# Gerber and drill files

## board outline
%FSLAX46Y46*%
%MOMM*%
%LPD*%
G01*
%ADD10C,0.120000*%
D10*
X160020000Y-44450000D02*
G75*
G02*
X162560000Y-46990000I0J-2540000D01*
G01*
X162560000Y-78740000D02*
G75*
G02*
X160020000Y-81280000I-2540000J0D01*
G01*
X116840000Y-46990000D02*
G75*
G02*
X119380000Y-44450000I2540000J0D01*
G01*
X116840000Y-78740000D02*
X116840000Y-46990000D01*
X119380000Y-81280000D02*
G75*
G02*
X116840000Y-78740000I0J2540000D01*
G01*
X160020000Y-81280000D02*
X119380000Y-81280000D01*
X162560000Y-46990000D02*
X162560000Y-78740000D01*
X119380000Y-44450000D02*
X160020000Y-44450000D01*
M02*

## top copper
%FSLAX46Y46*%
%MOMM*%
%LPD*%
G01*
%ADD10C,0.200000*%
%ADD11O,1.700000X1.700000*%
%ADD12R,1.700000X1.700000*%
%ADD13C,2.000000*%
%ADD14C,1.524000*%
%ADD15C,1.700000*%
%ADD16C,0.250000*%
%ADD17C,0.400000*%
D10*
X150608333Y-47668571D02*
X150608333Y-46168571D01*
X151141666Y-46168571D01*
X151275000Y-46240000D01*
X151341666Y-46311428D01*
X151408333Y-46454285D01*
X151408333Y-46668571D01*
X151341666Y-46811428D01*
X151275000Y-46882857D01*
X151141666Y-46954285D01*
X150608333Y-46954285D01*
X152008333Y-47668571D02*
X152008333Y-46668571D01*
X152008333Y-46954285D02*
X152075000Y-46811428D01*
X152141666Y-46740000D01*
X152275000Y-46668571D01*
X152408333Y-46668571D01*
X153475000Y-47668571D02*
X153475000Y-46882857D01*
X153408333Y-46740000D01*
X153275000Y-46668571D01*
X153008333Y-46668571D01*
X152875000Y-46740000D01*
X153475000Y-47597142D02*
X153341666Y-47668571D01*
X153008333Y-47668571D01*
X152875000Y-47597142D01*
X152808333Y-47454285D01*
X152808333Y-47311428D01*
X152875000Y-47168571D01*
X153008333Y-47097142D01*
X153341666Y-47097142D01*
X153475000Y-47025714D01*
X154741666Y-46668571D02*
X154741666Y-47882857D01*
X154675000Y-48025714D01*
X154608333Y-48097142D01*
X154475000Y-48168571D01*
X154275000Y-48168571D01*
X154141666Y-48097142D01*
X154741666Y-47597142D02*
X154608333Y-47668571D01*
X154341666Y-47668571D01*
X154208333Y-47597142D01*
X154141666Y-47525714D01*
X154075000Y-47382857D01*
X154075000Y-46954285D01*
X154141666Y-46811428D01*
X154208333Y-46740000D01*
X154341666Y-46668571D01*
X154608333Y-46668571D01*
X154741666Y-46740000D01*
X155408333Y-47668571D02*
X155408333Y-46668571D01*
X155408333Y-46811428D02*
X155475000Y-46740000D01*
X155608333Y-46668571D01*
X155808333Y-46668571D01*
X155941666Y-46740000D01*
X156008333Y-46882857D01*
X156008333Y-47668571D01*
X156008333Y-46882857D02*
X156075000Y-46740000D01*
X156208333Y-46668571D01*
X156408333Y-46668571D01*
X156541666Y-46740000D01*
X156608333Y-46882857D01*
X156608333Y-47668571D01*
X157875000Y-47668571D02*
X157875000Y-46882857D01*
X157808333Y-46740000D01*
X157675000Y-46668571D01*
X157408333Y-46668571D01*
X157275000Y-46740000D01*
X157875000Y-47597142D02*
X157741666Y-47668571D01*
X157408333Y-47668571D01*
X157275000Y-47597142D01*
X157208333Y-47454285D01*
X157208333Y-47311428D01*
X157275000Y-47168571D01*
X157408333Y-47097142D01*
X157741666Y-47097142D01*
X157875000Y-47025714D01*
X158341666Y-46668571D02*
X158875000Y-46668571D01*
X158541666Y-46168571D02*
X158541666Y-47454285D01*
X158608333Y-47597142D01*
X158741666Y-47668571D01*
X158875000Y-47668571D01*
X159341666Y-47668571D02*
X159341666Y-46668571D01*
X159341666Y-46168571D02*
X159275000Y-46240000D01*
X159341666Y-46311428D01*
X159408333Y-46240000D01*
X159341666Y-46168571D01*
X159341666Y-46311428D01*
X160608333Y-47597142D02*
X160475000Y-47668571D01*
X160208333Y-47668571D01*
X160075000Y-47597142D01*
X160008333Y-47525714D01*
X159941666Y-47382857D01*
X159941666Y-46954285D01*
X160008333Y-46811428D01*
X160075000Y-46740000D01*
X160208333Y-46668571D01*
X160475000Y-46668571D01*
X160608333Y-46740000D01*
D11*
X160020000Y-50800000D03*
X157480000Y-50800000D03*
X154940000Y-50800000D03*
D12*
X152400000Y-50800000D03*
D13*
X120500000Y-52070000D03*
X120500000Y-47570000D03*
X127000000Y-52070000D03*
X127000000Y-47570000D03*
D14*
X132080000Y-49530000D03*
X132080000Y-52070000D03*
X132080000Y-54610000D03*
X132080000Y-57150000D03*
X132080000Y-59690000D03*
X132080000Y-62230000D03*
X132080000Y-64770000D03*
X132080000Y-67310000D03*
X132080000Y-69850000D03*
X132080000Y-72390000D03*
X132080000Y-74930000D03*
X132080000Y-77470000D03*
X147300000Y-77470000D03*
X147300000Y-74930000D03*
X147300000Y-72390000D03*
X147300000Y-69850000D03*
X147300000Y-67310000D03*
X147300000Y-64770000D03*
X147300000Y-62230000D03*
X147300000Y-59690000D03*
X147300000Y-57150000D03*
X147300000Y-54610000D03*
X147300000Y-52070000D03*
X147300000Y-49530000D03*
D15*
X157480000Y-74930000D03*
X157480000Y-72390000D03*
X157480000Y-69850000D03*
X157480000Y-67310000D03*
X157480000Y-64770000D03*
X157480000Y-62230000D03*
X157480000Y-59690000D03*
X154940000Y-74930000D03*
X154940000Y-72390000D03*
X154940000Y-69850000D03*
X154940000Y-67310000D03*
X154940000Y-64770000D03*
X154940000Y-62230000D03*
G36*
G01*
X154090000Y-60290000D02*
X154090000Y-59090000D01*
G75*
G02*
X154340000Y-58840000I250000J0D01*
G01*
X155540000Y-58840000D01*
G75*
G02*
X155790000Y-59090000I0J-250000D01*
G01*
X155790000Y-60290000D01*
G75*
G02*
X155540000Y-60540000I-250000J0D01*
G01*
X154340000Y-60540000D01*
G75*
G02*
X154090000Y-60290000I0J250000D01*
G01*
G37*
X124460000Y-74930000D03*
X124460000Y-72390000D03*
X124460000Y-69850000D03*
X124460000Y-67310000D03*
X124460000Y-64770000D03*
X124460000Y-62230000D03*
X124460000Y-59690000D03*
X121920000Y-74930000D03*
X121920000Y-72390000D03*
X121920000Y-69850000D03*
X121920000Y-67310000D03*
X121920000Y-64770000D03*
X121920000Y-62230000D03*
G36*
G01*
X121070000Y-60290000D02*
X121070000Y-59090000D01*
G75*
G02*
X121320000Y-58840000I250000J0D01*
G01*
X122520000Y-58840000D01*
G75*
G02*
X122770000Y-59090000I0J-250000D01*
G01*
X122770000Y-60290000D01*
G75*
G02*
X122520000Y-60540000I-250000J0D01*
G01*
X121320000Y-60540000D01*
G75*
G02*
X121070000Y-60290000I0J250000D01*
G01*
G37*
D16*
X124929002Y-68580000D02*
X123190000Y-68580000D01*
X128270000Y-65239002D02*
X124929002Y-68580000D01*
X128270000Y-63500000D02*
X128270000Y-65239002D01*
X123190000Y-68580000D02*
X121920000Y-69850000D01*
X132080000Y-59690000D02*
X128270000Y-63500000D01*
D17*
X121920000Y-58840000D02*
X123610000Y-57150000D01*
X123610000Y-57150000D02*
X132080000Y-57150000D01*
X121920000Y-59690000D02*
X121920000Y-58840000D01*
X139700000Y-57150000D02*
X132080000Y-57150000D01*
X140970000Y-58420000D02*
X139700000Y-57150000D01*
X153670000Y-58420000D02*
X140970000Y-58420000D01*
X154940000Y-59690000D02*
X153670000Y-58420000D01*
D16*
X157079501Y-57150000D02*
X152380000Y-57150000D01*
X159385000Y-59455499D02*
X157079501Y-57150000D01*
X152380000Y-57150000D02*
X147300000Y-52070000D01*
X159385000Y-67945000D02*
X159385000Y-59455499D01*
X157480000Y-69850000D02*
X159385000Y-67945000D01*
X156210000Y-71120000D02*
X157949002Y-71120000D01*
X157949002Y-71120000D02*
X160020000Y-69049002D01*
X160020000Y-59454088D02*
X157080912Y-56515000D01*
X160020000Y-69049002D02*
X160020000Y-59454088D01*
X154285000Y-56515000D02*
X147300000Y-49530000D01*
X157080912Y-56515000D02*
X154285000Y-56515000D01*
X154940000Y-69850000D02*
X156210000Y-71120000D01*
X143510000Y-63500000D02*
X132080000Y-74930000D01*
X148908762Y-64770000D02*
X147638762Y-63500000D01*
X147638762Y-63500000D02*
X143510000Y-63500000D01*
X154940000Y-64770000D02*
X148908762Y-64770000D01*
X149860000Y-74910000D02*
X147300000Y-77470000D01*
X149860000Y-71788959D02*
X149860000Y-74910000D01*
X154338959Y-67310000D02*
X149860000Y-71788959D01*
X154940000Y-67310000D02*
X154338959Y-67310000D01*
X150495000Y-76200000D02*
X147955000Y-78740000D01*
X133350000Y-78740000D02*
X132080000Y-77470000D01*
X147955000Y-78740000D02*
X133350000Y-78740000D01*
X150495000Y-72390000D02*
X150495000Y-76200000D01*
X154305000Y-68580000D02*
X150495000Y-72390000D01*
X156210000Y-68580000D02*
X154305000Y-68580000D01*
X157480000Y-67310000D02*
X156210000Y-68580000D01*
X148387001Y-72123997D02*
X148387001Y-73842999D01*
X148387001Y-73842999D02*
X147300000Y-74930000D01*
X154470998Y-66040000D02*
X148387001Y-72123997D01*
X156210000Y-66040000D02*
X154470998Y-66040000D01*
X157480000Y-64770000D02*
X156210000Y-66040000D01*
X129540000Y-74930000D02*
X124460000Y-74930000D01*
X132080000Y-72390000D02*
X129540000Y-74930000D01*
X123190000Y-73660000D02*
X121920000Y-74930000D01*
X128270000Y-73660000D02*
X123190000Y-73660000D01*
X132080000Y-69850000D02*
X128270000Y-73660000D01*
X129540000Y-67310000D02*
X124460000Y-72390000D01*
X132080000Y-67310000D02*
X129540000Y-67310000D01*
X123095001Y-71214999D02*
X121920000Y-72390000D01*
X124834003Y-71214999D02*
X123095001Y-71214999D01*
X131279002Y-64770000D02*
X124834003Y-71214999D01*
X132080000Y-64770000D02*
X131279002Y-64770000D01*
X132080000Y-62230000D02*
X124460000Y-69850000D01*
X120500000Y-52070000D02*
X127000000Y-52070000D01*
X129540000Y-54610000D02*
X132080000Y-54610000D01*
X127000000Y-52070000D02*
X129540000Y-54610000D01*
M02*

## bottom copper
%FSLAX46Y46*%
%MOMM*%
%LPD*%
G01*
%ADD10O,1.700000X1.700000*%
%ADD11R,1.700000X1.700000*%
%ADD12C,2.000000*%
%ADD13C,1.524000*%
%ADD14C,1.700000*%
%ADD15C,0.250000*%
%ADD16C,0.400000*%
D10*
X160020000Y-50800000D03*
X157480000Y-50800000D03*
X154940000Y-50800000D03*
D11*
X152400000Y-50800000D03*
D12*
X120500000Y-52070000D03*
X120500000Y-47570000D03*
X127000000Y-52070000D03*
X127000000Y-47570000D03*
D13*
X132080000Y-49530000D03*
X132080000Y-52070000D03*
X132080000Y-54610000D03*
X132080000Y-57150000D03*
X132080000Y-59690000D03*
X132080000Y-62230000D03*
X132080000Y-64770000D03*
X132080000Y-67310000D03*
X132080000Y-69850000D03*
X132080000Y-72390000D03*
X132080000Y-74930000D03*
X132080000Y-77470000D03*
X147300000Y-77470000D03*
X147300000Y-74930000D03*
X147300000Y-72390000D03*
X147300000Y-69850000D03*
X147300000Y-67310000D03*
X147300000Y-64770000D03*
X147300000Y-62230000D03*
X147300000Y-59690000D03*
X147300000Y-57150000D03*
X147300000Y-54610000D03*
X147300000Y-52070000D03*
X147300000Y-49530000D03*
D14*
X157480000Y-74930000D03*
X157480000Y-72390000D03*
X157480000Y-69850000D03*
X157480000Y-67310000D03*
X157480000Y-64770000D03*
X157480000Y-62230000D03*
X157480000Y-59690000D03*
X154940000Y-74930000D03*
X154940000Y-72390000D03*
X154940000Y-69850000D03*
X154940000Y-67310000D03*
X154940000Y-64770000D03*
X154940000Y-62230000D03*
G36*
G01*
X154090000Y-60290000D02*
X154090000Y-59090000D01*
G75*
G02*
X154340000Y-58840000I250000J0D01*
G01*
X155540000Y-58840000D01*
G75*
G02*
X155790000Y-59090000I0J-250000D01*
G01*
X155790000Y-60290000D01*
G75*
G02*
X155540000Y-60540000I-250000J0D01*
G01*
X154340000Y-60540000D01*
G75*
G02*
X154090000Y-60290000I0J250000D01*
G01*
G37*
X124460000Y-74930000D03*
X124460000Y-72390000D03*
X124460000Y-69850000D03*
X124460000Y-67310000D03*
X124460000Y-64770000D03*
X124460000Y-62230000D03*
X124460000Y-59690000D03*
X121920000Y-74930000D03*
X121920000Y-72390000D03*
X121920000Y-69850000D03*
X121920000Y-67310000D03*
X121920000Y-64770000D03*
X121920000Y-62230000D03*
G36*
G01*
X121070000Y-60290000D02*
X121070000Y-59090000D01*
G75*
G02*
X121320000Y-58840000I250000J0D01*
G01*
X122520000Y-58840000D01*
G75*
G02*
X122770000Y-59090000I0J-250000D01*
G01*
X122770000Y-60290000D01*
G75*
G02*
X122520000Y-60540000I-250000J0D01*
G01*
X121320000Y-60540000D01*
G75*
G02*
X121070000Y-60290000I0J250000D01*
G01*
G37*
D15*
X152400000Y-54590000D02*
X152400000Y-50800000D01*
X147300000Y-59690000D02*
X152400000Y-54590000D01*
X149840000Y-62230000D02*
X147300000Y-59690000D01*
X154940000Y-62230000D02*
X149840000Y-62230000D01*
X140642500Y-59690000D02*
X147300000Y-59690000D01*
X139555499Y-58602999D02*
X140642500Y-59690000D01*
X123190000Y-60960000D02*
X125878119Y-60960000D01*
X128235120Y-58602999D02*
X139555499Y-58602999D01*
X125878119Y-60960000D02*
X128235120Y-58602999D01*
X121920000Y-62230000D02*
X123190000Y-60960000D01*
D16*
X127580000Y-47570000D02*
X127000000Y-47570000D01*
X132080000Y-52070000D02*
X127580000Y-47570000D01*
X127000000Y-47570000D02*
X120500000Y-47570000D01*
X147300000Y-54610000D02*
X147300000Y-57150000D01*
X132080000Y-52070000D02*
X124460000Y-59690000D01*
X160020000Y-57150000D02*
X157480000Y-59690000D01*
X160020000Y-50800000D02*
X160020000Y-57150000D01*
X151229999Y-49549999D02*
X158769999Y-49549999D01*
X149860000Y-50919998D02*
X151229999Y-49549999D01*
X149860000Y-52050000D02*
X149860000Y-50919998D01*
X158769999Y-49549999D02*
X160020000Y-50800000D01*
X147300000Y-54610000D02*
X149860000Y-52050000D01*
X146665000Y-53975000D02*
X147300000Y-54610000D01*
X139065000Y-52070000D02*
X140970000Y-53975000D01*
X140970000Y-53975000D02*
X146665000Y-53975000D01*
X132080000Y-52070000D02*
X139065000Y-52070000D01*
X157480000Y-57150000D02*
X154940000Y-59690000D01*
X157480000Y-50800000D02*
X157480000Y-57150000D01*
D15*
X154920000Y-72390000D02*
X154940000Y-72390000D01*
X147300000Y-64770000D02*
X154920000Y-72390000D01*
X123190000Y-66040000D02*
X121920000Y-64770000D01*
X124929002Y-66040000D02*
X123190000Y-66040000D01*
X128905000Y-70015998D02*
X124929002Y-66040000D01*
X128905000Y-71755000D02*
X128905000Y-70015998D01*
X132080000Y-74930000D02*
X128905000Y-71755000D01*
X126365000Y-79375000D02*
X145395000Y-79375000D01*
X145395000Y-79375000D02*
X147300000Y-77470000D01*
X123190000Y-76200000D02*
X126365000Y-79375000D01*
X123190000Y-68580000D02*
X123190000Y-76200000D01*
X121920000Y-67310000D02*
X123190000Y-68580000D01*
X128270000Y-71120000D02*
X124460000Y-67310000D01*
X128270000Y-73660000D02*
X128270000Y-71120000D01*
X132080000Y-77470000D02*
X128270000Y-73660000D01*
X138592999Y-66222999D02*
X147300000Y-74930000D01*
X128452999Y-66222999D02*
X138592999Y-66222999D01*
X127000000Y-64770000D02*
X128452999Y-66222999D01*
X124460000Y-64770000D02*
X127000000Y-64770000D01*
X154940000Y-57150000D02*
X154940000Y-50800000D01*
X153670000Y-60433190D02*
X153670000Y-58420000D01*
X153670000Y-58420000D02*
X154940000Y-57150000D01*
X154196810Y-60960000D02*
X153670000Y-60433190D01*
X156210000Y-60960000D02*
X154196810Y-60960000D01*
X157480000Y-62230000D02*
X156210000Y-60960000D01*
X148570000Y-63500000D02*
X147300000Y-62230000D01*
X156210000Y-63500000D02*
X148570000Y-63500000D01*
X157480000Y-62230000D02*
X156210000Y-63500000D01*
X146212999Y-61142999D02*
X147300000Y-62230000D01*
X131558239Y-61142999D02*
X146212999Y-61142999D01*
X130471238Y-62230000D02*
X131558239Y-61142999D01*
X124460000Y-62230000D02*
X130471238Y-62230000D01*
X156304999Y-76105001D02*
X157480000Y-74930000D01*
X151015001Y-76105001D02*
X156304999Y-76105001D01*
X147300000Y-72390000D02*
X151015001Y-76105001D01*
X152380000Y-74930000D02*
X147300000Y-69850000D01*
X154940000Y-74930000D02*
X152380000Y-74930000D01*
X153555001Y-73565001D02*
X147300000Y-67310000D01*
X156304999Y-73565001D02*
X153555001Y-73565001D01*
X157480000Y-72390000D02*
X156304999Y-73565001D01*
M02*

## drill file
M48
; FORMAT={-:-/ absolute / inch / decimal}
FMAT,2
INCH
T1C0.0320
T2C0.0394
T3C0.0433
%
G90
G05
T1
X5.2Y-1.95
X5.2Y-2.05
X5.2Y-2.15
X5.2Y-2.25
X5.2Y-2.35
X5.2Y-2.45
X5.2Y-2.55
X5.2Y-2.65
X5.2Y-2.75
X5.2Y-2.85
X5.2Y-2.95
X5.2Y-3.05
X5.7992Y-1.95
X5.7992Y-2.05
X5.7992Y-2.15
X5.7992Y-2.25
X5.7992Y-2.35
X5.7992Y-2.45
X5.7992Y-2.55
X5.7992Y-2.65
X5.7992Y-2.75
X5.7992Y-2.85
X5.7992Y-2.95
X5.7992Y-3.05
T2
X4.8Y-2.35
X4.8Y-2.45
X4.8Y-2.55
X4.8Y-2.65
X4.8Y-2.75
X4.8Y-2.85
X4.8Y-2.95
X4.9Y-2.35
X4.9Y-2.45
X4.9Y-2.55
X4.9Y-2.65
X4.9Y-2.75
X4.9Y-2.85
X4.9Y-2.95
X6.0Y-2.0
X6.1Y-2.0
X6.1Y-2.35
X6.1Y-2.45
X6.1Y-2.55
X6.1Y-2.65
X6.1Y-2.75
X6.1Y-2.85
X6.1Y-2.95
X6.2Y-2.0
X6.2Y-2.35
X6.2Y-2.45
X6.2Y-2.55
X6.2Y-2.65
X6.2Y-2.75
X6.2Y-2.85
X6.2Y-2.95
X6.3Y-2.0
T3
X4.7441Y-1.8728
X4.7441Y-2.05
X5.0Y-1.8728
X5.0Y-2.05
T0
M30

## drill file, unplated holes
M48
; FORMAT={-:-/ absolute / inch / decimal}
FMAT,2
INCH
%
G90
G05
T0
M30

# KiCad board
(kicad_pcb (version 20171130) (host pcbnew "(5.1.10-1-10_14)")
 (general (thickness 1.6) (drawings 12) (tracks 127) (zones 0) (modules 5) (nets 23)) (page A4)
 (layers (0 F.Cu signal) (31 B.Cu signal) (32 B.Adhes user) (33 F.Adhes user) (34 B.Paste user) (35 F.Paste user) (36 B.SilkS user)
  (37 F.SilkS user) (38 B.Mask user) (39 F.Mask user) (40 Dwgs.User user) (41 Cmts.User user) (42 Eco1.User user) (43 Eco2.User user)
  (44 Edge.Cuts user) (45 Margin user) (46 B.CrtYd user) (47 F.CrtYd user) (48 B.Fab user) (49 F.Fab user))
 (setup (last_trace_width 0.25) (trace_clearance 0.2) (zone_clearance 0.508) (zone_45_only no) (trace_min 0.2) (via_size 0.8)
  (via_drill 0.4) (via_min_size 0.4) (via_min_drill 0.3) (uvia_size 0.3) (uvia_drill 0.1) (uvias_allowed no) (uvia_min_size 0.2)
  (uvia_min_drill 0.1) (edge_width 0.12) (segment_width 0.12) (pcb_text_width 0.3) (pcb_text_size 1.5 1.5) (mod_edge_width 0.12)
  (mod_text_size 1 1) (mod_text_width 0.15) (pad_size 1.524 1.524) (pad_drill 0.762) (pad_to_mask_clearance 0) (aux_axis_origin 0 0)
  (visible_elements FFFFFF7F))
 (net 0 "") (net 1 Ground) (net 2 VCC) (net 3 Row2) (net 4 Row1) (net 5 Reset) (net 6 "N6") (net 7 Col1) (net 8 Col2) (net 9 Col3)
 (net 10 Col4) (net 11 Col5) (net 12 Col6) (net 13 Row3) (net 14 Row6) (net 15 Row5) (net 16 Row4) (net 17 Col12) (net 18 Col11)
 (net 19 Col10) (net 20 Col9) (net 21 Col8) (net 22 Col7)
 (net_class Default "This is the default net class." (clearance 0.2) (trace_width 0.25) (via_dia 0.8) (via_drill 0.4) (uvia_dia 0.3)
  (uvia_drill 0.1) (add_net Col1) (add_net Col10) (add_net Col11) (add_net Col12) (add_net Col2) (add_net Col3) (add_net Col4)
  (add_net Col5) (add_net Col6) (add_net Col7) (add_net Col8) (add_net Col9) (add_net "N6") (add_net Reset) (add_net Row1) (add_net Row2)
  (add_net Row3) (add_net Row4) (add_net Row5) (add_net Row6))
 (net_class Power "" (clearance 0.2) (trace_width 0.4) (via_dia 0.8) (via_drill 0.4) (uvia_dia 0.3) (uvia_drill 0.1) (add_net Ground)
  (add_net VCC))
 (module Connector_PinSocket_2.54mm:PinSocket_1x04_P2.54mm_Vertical (layer F.Cu) (at 152.4 50.8 90)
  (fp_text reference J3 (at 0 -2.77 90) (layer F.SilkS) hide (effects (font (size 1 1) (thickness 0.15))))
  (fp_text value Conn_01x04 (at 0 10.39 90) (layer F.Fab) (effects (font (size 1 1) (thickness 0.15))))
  (pad 4 thru_hole oval (at 0 7.62 90) (size 1.7 1.7) (drill 1) (layers *.Cu *.Mask) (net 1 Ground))
  (pad 3 thru_hole oval (at 0 5.08 90) (size 1.7 1.7) (drill 1) (layers *.Cu *.Mask) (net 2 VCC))
  (pad 2 thru_hole oval (at 0 2.54 90) (size 1.7 1.7) (drill 1) (layers *.Cu *.Mask) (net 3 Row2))
  (pad 1 thru_hole rect (at 0 0 90) (size 1.7 1.7) (drill 1) (layers *.Cu *.Mask) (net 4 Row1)))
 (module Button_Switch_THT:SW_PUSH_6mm (layer F.Cu) (at 127 52.07 180)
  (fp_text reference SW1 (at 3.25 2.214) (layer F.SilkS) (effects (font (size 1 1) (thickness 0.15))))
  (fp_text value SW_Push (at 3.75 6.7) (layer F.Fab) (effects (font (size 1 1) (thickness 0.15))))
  (pad 1 thru_hole circle (at 6.5 0 270) (size 2 2) (drill 1.1) (layers *.Cu *.Mask) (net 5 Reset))
  (pad 2 thru_hole circle (at 6.5 4.5 270) (size 2 2) (drill 1.1) (layers *.Cu *.Mask) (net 1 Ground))
  (pad 1 thru_hole circle (at 0 0 270) (size 2 2) (drill 1.1) (layers *.Cu *.Mask) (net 5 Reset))
  (pad 2 thru_hole circle (at 0 4.5 270) (size 2 2) (drill 1.1) (layers *.Cu *.Mask) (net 1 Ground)))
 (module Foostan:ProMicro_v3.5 (layer F.Cu) (at 139.6886 64.008)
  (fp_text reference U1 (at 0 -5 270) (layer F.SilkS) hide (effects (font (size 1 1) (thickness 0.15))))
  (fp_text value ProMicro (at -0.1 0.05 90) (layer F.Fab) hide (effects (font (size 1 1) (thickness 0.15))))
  (pad 24 thru_hole circle (at -7.6086 -14.478) (size 1.524 1.524) (drill 0.8128) (layers *.Cu F.SilkS B.Mask) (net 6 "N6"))
  (pad 23 thru_hole circle (at -7.6086 -11.938) (size 1.524 1.524) (drill 0.8128) (layers *.Cu F.SilkS B.Mask) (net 1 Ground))
  (pad 22 thru_hole circle (at -7.6086 -9.398) (size 1.524 1.524) (drill 0.8128) (layers *.Cu F.SilkS B.Mask) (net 5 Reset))
  (pad 21 thru_hole circle (at -7.6086 -6.858) (size 1.524 1.524) (drill 0.8128) (layers *.Cu F.SilkS B.Mask) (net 2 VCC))
  (pad 20 thru_hole circle (at -7.6086 -4.318) (size 1.524 1.524) (drill 0.8128) (layers *.Cu F.SilkS B.Mask) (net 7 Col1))
  (pad 19 thru_hole circle (at -7.6086 -1.778) (size 1.524 1.524) (drill 0.8128) (layers *.Cu F.SilkS B.Mask) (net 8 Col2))
  (pad 18 thru_hole circle (at -7.6086 0.762) (size 1.524 1.524) (drill 0.8128) (layers *.Cu F.SilkS B.Mask) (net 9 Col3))
  (pad 17 thru_hole circle (at -7.6086 3.302) (size 1.524 1.524) (drill 0.8128) (layers *.Cu F.SilkS B.Mask) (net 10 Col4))
  (pad 16 thru_hole circle (at -7.6086 5.842) (size 1.524 1.524) (drill 0.8128) (layers *.Cu F.SilkS B.Mask) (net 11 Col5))
  (pad 15 thru_hole circle (at -7.6086 8.382) (size 1.524 1.524) (drill 0.8128) (layers *.Cu F.SilkS B.Mask) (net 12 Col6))
  (pad 14 thru_hole circle (at -7.6086 10.922) (size 1.524 1.524) (drill 0.8128) (layers *.Cu F.SilkS B.Mask) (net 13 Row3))
  (pad 13 thru_hole circle (at -7.6086 13.462) (size 1.524 1.524) (drill 0.8128) (layers *.Cu F.SilkS B.Mask) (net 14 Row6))
  (pad 12 thru_hole circle (at 7.6114 13.462) (size 1.524 1.524) (drill 0.8128) (layers *.Cu F.SilkS B.Mask) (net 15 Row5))
  (pad 11 thru_hole circle (at 7.6114 10.922) (size 1.524 1.524) (drill 0.8128) (layers *.Cu F.SilkS B.Mask) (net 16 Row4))
  (pad 10 thru_hole circle (at 7.6114 8.382) (size 1.524 1.524) (drill 0.8128) (layers *.Cu F.SilkS B.Mask) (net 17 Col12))
  (pad 9 thru_hole circle (at 7.6114 5.842) (size 1.524 1.524) (drill 0.8128) (layers *.Cu F.SilkS B.Mask) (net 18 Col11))
  (pad 8 thru_hole circle (at 7.6114 3.302) (size 1.524 1.524) (drill 0.8128) (layers *.Cu F.SilkS B.Mask) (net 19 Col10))
  (pad 7 thru_hole circle (at 7.6114 0.762) (size 1.524 1.524) (drill 0.8128) (layers *.Cu F.SilkS B.Mask) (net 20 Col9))
  (pad 6 thru_hole circle (at 7.6114 -1.778) (size 1.524 1.524) (drill 0.8128) (layers *.Cu F.SilkS B.Mask) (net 3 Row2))
  (pad 5 thru_hole circle (at 7.6114 -4.318) (size 1.524 1.524) (drill 0.8128) (layers *.Cu F.SilkS B.Mask) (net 4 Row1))
  (pad 4 thru_hole circle (at 7.6114 -6.858) (size 1.524 1.524) (drill 0.8128) (layers *.Cu F.SilkS B.Mask) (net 1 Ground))
  (pad 3 thru_hole circle (at 7.6114 -9.398) (size 1.524 1.524) (drill 0.8128) (layers *.Cu F.SilkS B.Mask) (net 1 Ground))
  (pad 2 thru_hole circle (at 7.6114 -11.938) (size 1.524 1.524) (drill 0.8128) (layers *.Cu F.SilkS B.Mask) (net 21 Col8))
  (pad 1 thru_hole circle (at 7.6114 -14.478) (size 1.524 1.524) (drill 0.8128) (layers *.Cu F.SilkS B.Mask) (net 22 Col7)))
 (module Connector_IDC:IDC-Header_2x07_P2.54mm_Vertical (layer F.Cu) (at 154.94 59.69)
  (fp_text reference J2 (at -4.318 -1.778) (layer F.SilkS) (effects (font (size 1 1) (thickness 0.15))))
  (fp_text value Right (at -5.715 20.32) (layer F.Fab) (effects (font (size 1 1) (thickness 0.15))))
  (pad 14 thru_hole circle (at 2.54 15.24) (size 1.7 1.7) (drill 1) (layers *.Cu *.Mask) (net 17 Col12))
  (pad 12 thru_hole circle (at 2.54 12.7) (size 1.7 1.7) (drill 1) (layers *.Cu *.Mask) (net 19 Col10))
  (pad 10 thru_hole circle (at 2.54 10.16) (size 1.7 1.7) (drill 1) (layers *.Cu *.Mask) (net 21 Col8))
  (pad 8 thru_hole circle (at 2.54 7.62) (size 1.7 1.7) (drill 1) (layers *.Cu *.Mask) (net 14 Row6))
  (pad 6 thru_hole circle (at 2.54 5.08) (size 1.7 1.7) (drill 1) (layers *.Cu *.Mask) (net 16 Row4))
  (pad 4 thru_hole circle (at 2.54 2.54) (size 1.7 1.7) (drill 1) (layers *.Cu *.Mask) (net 3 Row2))
  (pad 2 thru_hole circle (at 2.54 0) (size 1.7 1.7) (drill 1) (layers *.Cu *.Mask) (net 1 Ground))
  (pad 13 thru_hole circle (at 0 15.24) (size 1.7 1.7) (drill 1) (layers *.Cu *.Mask) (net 18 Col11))
  (pad 11 thru_hole circle (at 0 12.7) (size 1.7 1.7) (drill 1) (layers *.Cu *.Mask) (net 20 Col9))
  (pad 9 thru_hole circle (at 0 10.16) (size 1.7 1.7) (drill 1) (layers *.Cu *.Mask) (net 22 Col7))
  (pad 7 thru_hole circle (at 0 7.62) (size 1.7 1.7) (drill 1) (layers *.Cu *.Mask) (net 15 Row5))
  (pad 5 thru_hole circle (at 0 5.08) (size 1.7 1.7) (drill 1) (layers *.Cu *.Mask) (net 13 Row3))
  (pad 3 thru_hole circle (at 0 2.54) (size 1.7 1.7) (drill 1) (layers *.Cu *.Mask) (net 4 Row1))
  (pad 1 thru_hole roundrect (at 0 0) (size 1.7 1.7) (drill 1) (layers *.Cu *.Mask) (roundrect_rratio 0.1470588235294118) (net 2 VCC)))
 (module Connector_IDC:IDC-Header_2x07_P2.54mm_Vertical (layer F.Cu) (at 121.92 59.69)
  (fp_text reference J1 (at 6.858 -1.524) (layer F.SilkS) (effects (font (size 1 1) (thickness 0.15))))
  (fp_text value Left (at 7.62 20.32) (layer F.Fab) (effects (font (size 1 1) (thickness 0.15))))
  (pad 14 thru_hole circle (at 2.54 15.24) (size 1.7 1.7) (drill 1) (layers *.Cu *.Mask) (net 12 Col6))
  (pad 12 thru_hole circle (at 2.54 12.7) (size 1.7 1.7) (drill 1) (layers *.Cu *.Mask) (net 10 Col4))
  (pad 10 thru_hole circle (at 2.54 10.16) (size 1.7 1.7) (drill 1) (layers *.Cu *.Mask) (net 8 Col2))
  (pad 8 thru_hole circle (at 2.54 7.62) (size 1.7 1.7) (drill 1) (layers *.Cu *.Mask) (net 14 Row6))
  (pad 6 thru_hole circle (at 2.54 5.08) (size 1.7 1.7) (drill 1) (layers *.Cu *.Mask) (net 16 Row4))
  (pad 4 thru_hole circle (at 2.54 2.54) (size 1.7 1.7) (drill 1) (layers *.Cu *.Mask) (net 3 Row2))
  (pad 2 thru_hole circle (at 2.54 0) (size 1.7 1.7) (drill 1) (layers *.Cu *.Mask) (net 1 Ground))
  (pad 13 thru_hole circle (at 0 15.24) (size 1.7 1.7) (drill 1) (layers *.Cu *.Mask) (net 11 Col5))
  (pad 11 thru_hole circle (at 0 12.7) (size 1.7 1.7) (drill 1) (layers *.Cu *.Mask) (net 9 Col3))
  (pad 9 thru_hole circle (at 0 10.16) (size 1.7 1.7) (drill 1) (layers *.Cu *.Mask) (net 7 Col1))
  (pad 7 thru_hole circle (at 0 7.62) (size 1.7 1.7) (drill 1) (layers *.Cu *.Mask) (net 15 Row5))
  (pad 5 thru_hole circle (at 0 5.08) (size 1.7 1.7) (drill 1) (layers *.Cu *.Mask) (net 13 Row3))
  (pad 3 thru_hole circle (at 0 2.54) (size 1.7 1.7) (drill 1) (layers *.Cu *.Mask) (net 4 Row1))
  (pad 1 thru_hole roundrect (at 0 0) (size 1.7 1.7) (drill 1) (layers *.Cu *.Mask) (roundrect_rratio 0.1470588235294118) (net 2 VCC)))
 (gr_arc (start 160.02 46.99) (end 162.56 46.99) (angle -90) (layer Edge.Cuts) (width 0.12))
 (gr_arc (start 160.02 78.74) (end 160.02 81.28) (angle -90) (layer Edge.Cuts) (width 0.12))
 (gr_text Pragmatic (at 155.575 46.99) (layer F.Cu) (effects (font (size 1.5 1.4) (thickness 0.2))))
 (gr_arc (start 119.38 46.99) (end 119.38 44.45) (angle -90) (layer Edge.Cuts) (width 0.12))
 (gr_line (start 116.84 78.74) (end 116.84 46.99) (layer Edge.Cuts) (width 0.12))
 (gr_arc (start 119.38 78.74) (end 116.84 78.74) (angle -90) (layer Edge.Cuts) (width 0.12))
 (gr_line (start 160.02 81.28) (end 119.38 81.28) (layer Edge.Cuts) (width 0.12))
 (gr_line (start 162.56 46.99) (end 162.56 78.74) (layer Edge.Cuts) (width 0.12))
 (gr_line (start 119.38 44.45) (end 160.02 44.45) (layer Edge.Cuts) (width 0.12))
 (segment (start 152.4 54.59) (end 152.4 50.8) (width 0.25) (layer B.Cu) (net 4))
 (segment (start 147.3 59.69) (end 152.4 54.59) (width 0.25) (layer B.Cu) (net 4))
 (segment (start 149.84 62.23) (end 147.3 59.69) (width 0.25) (layer B.Cu) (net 4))
 (segment (start 154.94 62.23) (end 149.84 62.23) (width 0.25) (layer B.Cu) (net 4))
 (segment (start 140.6425 59.69) (end 147.3 59.69) (width 0.25) (layer B.Cu) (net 4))
 (segment (start 139.555499 58.602999) (end 140.6425 59.69) (width 0.25) (layer B.Cu) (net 4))
 (segment (start 123.19 60.96) (end 125.878119 60.96) (width 0.25) (layer B.Cu) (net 4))
 (segment (start 128.23512 58.602999) (end 139.555499 58.602999) (width 0.25) (layer B.Cu) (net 4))
 (segment (start 125.878119 60.96) (end 128.23512 58.602999) (width 0.25) (layer B.Cu) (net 4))
 (segment (start 121.92 62.23) (end 123.19 60.96) (width 0.25) (layer B.Cu) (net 4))
 (segment (start 124.929002 68.58) (end 123.19 68.58) (width 0.25) (layer F.Cu) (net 7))
 (segment (start 128.27 65.239002) (end 124.929002 68.58) (width 0.25) (layer F.Cu) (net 7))
 (segment (start 128.27 63.5) (end 128.27 65.239002) (width 0.25) (layer F.Cu) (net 7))
 (segment (start 123.19 68.58) (end 121.92 69.85) (width 0.25) (layer F.Cu) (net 7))
 (segment (start 132.08 59.69) (end 128.27 63.5) (width 0.25) (layer F.Cu) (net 7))
 (segment (start 127.58 47.57) (end 127 47.57) (width 0.4) (layer B.Cu) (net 1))
 (segment (start 132.08 52.07) (end 127.58 47.57) (width 0.4) (layer B.Cu) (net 1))
 (segment (start 127 47.57) (end 120.5 47.57) (width 0.4) (layer B.Cu) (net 1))
 (segment (start 147.3 54.61) (end 147.3 57.15) (width 0.4) (layer B.Cu) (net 1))
 (segment (start 132.08 52.07) (end 124.46 59.69) (width 0.4) (layer B.Cu) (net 1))
 (segment (start 160.02 57.15) (end 157.48 59.69) (width 0.4) (layer B.Cu) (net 1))
 (segment (start 160.02 50.8) (end 160.02 57.15) (width 0.4) (layer B.Cu) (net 1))
 (segment (start 151.229999 49.549999) (end 158.769999 49.549999) (width 0.4) (layer B.Cu) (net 1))
 (segment (start 149.86 50.919998) (end 151.229999 49.549999) (width 0.4) (layer B.Cu) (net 1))
 (segment (start 149.86 52.05) (end 149.86 50.919998) (width 0.4) (layer B.Cu) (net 1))
 (segment (start 158.769999 49.549999) (end 160.02 50.8) (width 0.4) (layer B.Cu) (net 1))
 (segment (start 147.3 54.61) (end 149.86 52.05) (width 0.4) (layer B.Cu) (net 1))
 (segment (start 146.665 53.975) (end 147.3 54.61) (width 0.4) (layer B.Cu) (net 1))
 (segment (start 139.065 52.07) (end 140.97 53.975) (width 0.4) (layer B.Cu) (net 1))
 (segment (start 140.97 53.975) (end 146.665 53.975) (width 0.4) (layer B.Cu) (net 1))
 (segment (start 132.08 52.07) (end 139.065 52.07) (width 0.4) (layer B.Cu) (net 1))
 (segment (start 157.48 57.15) (end 154.94 59.69) (width 0.4) (layer B.Cu) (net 2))
 (segment (start 157.48 50.8) (end 157.48 57.15) (width 0.4) (layer B.Cu) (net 2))
 (segment (start 121.92 58.84) (end 123.61 57.15) (width 0.4) (layer F.Cu) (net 2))
 (segment (start 123.61 57.15) (end 132.08 57.15) (width 0.4) (layer F.Cu) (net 2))
 (segment (start 121.92 59.69) (end 121.92 58.84) (width 0.4) (layer F.Cu) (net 2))
 (segment (start 139.7 57.15) (end 132.08 57.15) (width 0.4) (layer F.Cu) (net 2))
 (segment (start 140.97 58.42) (end 139.7 57.15) (width 0.4) (layer F.Cu) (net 2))
 (segment (start 153.67 58.42) (end 140.97 58.42) (width 0.4) (layer F.Cu) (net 2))
 (segment (start 154.94 59.69) (end 153.67 58.42) (width 0.4) (layer F.Cu) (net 2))
 (segment (start 154.92 72.39) (end 154.94 72.39) (width 0.25) (layer B.Cu) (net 20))
 (segment (start 147.3 64.77) (end 154.92 72.39) (width 0.25) (layer B.Cu) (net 20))
 (segment (start 157.079501 57.15) (end 152.38 57.15) (width 0.25) (layer F.Cu) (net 21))
 (segment (start 159.385 59.455499) (end 157.079501 57.15) (width 0.25) (layer F.Cu) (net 21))
 (segment (start 152.38 57.15) (end 147.3 52.07) (width 0.25) (layer F.Cu) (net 21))
 (segment (start 159.385 67.945) (end 159.385 59.455499) (width 0.25) (layer F.Cu) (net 21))
 (segment (start 157.48 69.85) (end 159.385 67.945) (width 0.25) (layer F.Cu) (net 21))
 (segment (start 156.21 71.12) (end 157.949002 71.12) (width 0.25) (layer F.Cu) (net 22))
 (segment (start 157.949002 71.12) (end 160.02 69.049002) (width 0.25) (layer F.Cu) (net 22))
 (segment (start 160.02 59.454088) (end 157.080912 56.515) (width 0.25) (layer F.Cu) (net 22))
 (segment (start 160.02 69.049002) (end 160.02 59.454088) (width 0.25) (layer F.Cu) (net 22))
 (segment (start 154.285 56.515) (end 147.3 49.53) (width 0.25) (layer F.Cu) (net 22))
 (segment (start 157.080912 56.515) (end 154.285 56.515) (width 0.25) (layer F.Cu) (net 22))
 (segment (start 154.94 69.85) (end 156.21 71.12) (width 0.25) (layer F.Cu) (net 22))
 (segment (start 143.51 63.5) (end 132.08 74.93) (width 0.25) (layer F.Cu) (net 13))
 (segment (start 148.908762 64.77) (end 147.638762 63.5) (width 0.25) (layer F.Cu) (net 13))
 (segment (start 147.638762 63.5) (end 143.51 63.5) (width 0.25) (layer F.Cu) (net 13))
 (segment (start 154.94 64.77) (end 148.908762 64.77) (width 0.25) (layer F.Cu) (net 13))
 (segment (start 123.19 66.04) (end 121.92 64.77) (width 0.25) (layer B.Cu) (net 13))
 (segment (start 124.929002 66.04) (end 123.19 66.04) (width 0.25) (layer B.Cu) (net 13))
 (segment (start 128.905 70.015998) (end 124.929002 66.04) (width 0.25) (layer B.Cu) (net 13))
 (segment (start 128.905 71.755) (end 128.905 70.015998) (width 0.25) (layer B.Cu) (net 13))
 (segment (start 132.08 74.93) (end 128.905 71.755) (width 0.25) (layer B.Cu) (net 13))
 (segment (start 149.86 74.91) (end 147.3 77.47) (width 0.25) (layer F.Cu) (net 15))
 (segment (start 149.86 71.788959) (end 149.86 74.91) (width 0.25) (layer F.Cu) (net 15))
 (segment (start 154.338959 67.31) (end 149.86 71.788959) (width 0.25) (layer F.Cu) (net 15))
 (segment (start 154.94 67.31) (end 154.338959 67.31) (width 0.25) (layer F.Cu) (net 15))
 (segment (start 126.365 79.375) (end 145.395 79.375) (width 0.25) (layer B.Cu) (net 15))
 (segment (start 145.395 79.375) (end 147.3 77.47) (width 0.25) (layer B.Cu) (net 15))
 (segment (start 123.19 76.2) (end 126.365 79.375) (width 0.25) (layer B.Cu) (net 15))
 (segment (start 123.19 68.58) (end 123.19 76.2) (width 0.25) (layer B.Cu) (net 15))
 (segment (start 121.92 67.31) (end 123.19 68.58) (width 0.25) (layer B.Cu) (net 15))
 (segment (start 150.495 76.2) (end 147.955 78.74) (width 0.25) (layer F.Cu) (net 14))
 (segment (start 133.35 78.74) (end 132.08 77.47) (width 0.25) (layer F.Cu) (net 14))
 (segment (start 147.955 78.74) (end 133.35 78.74) (width 0.25) (layer F.Cu) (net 14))
 (segment (start 150.495 72.39) (end 150.495 76.2) (width 0.25) (layer F.Cu) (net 14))
 (segment (start 154.305 68.58) (end 150.495 72.39) (width 0.25) (layer F.Cu) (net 14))
 (segment (start 156.21 68.58) (end 154.305 68.58) (width 0.25) (layer F.Cu) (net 14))
 (segment (start 157.48 67.31) (end 156.21 68.58) (width 0.25) (layer F.Cu) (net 14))
 (segment (start 128.27 71.12) (end 124.46 67.31) (width 0.25) (layer B.Cu) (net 14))
 (segment (start 128.27 73.66) (end 128.27 71.12) (width 0.25) (layer B.Cu) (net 14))
 (segment (start 132.08 77.47) (end 128.27 73.66) (width 0.25) (layer B.Cu) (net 14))
 (segment (start 148.387001 72.123997) (end 148.387001 73.842999) (width 0.25) (layer F.Cu) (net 16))
 (segment (start 148.387001 73.842999) (end 147.3 74.93) (width 0.25) (layer F.Cu) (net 16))
 (segment (start 154.470998 66.04) (end 148.387001 72.123997) (width 0.25) (layer F.Cu) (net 16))
 (segment (start 156.21 66.04) (end 154.470998 66.04) (width 0.25) (layer F.Cu) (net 16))
 (segment (start 157.48 64.77) (end 156.21 66.04) (width 0.25) (layer F.Cu) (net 16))
 (segment (start 138.592999 66.222999) (end 147.3 74.93) (width 0.25) (layer B.Cu) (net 16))
 (segment (start 128.452999 66.222999) (end 138.592999 66.222999) (width 0.25) (layer B.Cu) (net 16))
 (segment (start 127 64.77) (end 128.452999 66.222999) (width 0.25) (layer B.Cu) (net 16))
 (segment (start 124.46 64.77) (end 127 64.77) (width 0.25) (layer B.Cu) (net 16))
 (segment (start 129.54 74.93) (end 124.46 74.93) (width 0.25) (layer F.Cu) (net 12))
 (segment (start 132.08 72.39) (end 129.54 74.93) (width 0.25) (layer F.Cu) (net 12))
 (segment (start 123.19 73.66) (end 121.92 74.93) (width 0.25) (layer F.Cu) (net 11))
 (segment (start 128.27 73.66) (end 123.19 73.66) (width 0.25) (layer F.Cu) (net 11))
 (segment (start 132.08 69.85) (end 128.27 73.66) (width 0.25) (layer F.Cu) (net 11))
 (segment (start 129.54 67.31) (end 124.46 72.39) (width 0.25) (layer F.Cu) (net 10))
 (segment (start 132.08 67.31) (end 129.54 67.31) (width 0.25) (layer F.Cu) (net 10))
 (segment (start 123.095001 71.214999) (end 121.92 72.39) (width 0.25) (layer F.Cu) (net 9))
 (segment (start 124.834003 71.214999) (end 123.095001 71.214999) (width 0.25) (layer F.Cu) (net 9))
 (segment (start 131.279002 64.77) (end 124.834003 71.214999) (width 0.25) (layer F.Cu) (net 9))
 (segment (start 132.08 64.77) (end 131.279002 64.77) (width 0.25) (layer F.Cu) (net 9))
 (segment (start 132.08 62.23) (end 124.46 69.85) (width 0.25) (layer F.Cu) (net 8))
 (segment (start 154.94 57.15) (end 154.94 50.8) (width 0.25) (layer B.Cu) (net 3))
 (segment (start 153.67 60.43319) (end 153.67 58.42) (width 0.25) (layer B.Cu) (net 3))
 (segment (start 153.67 58.42) (end 154.94 57.15) (width 0.25) (layer B.Cu) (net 3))
 (segment (start 154.19681 60.96) (end 153.67 60.43319) (width 0.25) (layer B.Cu) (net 3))
 (segment (start 156.21 60.96) (end 154.19681 60.96) (width 0.25) (layer B.Cu) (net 3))
 (segment (start 157.48 62.23) (end 156.21 60.96) (width 0.25) (layer B.Cu) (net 3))
 (segment (start 148.57 63.5) (end 147.3 62.23) (width 0.25) (layer B.Cu) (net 3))
 (segment (start 156.21 63.5) (end 148.57 63.5) (width 0.25) (layer B.Cu) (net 3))
 (segment (start 157.48 62.23) (end 156.21 63.5) (width 0.25) (layer B.Cu) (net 3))
 (segment (start 146.212999 61.142999) (end 147.3 62.23) (width 0.25) (layer B.Cu) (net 3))
 (segment (start 131.558239 61.142999) (end 146.212999 61.142999) (width 0.25) (layer B.Cu) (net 3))
 (segment (start 130.471238 62.23) (end 131.558239 61.142999) (width 0.25) (layer B.Cu) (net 3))
 (segment (start 124.46 62.23) (end 130.471238 62.23) (width 0.25) (layer B.Cu) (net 3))
 (segment (start 120.5 52.07) (end 127 52.07) (width 0.25) (layer F.Cu) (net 5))
 (segment (start 129.54 54.61) (end 132.08 54.61) (width 0.25) (layer F.Cu) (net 5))
 (segment (start 127 52.07) (end 129.54 54.61) (width 0.25) (layer F.Cu) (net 5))
 (segment (start 156.304999 76.105001) (end 157.48 74.93) (width 0.25) (layer B.Cu) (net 17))
 (segment (start 151.015001 76.105001) (end 156.304999 76.105001) (width 0.25) (layer B.Cu) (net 17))
 (segment (start 147.3 72.39) (end 151.015001 76.105001) (width 0.25) (layer B.Cu) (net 17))
 (segment (start 152.38 74.93) (end 147.3 69.85) (width 0.25) (layer B.Cu) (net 18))
 (segment (start 154.94 74.93) (end 152.38 74.93) (width 0.25) (layer B.Cu) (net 18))
 (segment (start 153.555001 73.565001) (end 147.3 67.31) (width 0.25) (layer B.Cu) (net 19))
 (segment (start 156.304999 73.565001) (end 153.555001 73.565001) (width 0.25) (layer B.Cu) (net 19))
 (segment (start 157.48 72.39) (end 156.304999 73.565001) (width 0.25) (layer B.Cu) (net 19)))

